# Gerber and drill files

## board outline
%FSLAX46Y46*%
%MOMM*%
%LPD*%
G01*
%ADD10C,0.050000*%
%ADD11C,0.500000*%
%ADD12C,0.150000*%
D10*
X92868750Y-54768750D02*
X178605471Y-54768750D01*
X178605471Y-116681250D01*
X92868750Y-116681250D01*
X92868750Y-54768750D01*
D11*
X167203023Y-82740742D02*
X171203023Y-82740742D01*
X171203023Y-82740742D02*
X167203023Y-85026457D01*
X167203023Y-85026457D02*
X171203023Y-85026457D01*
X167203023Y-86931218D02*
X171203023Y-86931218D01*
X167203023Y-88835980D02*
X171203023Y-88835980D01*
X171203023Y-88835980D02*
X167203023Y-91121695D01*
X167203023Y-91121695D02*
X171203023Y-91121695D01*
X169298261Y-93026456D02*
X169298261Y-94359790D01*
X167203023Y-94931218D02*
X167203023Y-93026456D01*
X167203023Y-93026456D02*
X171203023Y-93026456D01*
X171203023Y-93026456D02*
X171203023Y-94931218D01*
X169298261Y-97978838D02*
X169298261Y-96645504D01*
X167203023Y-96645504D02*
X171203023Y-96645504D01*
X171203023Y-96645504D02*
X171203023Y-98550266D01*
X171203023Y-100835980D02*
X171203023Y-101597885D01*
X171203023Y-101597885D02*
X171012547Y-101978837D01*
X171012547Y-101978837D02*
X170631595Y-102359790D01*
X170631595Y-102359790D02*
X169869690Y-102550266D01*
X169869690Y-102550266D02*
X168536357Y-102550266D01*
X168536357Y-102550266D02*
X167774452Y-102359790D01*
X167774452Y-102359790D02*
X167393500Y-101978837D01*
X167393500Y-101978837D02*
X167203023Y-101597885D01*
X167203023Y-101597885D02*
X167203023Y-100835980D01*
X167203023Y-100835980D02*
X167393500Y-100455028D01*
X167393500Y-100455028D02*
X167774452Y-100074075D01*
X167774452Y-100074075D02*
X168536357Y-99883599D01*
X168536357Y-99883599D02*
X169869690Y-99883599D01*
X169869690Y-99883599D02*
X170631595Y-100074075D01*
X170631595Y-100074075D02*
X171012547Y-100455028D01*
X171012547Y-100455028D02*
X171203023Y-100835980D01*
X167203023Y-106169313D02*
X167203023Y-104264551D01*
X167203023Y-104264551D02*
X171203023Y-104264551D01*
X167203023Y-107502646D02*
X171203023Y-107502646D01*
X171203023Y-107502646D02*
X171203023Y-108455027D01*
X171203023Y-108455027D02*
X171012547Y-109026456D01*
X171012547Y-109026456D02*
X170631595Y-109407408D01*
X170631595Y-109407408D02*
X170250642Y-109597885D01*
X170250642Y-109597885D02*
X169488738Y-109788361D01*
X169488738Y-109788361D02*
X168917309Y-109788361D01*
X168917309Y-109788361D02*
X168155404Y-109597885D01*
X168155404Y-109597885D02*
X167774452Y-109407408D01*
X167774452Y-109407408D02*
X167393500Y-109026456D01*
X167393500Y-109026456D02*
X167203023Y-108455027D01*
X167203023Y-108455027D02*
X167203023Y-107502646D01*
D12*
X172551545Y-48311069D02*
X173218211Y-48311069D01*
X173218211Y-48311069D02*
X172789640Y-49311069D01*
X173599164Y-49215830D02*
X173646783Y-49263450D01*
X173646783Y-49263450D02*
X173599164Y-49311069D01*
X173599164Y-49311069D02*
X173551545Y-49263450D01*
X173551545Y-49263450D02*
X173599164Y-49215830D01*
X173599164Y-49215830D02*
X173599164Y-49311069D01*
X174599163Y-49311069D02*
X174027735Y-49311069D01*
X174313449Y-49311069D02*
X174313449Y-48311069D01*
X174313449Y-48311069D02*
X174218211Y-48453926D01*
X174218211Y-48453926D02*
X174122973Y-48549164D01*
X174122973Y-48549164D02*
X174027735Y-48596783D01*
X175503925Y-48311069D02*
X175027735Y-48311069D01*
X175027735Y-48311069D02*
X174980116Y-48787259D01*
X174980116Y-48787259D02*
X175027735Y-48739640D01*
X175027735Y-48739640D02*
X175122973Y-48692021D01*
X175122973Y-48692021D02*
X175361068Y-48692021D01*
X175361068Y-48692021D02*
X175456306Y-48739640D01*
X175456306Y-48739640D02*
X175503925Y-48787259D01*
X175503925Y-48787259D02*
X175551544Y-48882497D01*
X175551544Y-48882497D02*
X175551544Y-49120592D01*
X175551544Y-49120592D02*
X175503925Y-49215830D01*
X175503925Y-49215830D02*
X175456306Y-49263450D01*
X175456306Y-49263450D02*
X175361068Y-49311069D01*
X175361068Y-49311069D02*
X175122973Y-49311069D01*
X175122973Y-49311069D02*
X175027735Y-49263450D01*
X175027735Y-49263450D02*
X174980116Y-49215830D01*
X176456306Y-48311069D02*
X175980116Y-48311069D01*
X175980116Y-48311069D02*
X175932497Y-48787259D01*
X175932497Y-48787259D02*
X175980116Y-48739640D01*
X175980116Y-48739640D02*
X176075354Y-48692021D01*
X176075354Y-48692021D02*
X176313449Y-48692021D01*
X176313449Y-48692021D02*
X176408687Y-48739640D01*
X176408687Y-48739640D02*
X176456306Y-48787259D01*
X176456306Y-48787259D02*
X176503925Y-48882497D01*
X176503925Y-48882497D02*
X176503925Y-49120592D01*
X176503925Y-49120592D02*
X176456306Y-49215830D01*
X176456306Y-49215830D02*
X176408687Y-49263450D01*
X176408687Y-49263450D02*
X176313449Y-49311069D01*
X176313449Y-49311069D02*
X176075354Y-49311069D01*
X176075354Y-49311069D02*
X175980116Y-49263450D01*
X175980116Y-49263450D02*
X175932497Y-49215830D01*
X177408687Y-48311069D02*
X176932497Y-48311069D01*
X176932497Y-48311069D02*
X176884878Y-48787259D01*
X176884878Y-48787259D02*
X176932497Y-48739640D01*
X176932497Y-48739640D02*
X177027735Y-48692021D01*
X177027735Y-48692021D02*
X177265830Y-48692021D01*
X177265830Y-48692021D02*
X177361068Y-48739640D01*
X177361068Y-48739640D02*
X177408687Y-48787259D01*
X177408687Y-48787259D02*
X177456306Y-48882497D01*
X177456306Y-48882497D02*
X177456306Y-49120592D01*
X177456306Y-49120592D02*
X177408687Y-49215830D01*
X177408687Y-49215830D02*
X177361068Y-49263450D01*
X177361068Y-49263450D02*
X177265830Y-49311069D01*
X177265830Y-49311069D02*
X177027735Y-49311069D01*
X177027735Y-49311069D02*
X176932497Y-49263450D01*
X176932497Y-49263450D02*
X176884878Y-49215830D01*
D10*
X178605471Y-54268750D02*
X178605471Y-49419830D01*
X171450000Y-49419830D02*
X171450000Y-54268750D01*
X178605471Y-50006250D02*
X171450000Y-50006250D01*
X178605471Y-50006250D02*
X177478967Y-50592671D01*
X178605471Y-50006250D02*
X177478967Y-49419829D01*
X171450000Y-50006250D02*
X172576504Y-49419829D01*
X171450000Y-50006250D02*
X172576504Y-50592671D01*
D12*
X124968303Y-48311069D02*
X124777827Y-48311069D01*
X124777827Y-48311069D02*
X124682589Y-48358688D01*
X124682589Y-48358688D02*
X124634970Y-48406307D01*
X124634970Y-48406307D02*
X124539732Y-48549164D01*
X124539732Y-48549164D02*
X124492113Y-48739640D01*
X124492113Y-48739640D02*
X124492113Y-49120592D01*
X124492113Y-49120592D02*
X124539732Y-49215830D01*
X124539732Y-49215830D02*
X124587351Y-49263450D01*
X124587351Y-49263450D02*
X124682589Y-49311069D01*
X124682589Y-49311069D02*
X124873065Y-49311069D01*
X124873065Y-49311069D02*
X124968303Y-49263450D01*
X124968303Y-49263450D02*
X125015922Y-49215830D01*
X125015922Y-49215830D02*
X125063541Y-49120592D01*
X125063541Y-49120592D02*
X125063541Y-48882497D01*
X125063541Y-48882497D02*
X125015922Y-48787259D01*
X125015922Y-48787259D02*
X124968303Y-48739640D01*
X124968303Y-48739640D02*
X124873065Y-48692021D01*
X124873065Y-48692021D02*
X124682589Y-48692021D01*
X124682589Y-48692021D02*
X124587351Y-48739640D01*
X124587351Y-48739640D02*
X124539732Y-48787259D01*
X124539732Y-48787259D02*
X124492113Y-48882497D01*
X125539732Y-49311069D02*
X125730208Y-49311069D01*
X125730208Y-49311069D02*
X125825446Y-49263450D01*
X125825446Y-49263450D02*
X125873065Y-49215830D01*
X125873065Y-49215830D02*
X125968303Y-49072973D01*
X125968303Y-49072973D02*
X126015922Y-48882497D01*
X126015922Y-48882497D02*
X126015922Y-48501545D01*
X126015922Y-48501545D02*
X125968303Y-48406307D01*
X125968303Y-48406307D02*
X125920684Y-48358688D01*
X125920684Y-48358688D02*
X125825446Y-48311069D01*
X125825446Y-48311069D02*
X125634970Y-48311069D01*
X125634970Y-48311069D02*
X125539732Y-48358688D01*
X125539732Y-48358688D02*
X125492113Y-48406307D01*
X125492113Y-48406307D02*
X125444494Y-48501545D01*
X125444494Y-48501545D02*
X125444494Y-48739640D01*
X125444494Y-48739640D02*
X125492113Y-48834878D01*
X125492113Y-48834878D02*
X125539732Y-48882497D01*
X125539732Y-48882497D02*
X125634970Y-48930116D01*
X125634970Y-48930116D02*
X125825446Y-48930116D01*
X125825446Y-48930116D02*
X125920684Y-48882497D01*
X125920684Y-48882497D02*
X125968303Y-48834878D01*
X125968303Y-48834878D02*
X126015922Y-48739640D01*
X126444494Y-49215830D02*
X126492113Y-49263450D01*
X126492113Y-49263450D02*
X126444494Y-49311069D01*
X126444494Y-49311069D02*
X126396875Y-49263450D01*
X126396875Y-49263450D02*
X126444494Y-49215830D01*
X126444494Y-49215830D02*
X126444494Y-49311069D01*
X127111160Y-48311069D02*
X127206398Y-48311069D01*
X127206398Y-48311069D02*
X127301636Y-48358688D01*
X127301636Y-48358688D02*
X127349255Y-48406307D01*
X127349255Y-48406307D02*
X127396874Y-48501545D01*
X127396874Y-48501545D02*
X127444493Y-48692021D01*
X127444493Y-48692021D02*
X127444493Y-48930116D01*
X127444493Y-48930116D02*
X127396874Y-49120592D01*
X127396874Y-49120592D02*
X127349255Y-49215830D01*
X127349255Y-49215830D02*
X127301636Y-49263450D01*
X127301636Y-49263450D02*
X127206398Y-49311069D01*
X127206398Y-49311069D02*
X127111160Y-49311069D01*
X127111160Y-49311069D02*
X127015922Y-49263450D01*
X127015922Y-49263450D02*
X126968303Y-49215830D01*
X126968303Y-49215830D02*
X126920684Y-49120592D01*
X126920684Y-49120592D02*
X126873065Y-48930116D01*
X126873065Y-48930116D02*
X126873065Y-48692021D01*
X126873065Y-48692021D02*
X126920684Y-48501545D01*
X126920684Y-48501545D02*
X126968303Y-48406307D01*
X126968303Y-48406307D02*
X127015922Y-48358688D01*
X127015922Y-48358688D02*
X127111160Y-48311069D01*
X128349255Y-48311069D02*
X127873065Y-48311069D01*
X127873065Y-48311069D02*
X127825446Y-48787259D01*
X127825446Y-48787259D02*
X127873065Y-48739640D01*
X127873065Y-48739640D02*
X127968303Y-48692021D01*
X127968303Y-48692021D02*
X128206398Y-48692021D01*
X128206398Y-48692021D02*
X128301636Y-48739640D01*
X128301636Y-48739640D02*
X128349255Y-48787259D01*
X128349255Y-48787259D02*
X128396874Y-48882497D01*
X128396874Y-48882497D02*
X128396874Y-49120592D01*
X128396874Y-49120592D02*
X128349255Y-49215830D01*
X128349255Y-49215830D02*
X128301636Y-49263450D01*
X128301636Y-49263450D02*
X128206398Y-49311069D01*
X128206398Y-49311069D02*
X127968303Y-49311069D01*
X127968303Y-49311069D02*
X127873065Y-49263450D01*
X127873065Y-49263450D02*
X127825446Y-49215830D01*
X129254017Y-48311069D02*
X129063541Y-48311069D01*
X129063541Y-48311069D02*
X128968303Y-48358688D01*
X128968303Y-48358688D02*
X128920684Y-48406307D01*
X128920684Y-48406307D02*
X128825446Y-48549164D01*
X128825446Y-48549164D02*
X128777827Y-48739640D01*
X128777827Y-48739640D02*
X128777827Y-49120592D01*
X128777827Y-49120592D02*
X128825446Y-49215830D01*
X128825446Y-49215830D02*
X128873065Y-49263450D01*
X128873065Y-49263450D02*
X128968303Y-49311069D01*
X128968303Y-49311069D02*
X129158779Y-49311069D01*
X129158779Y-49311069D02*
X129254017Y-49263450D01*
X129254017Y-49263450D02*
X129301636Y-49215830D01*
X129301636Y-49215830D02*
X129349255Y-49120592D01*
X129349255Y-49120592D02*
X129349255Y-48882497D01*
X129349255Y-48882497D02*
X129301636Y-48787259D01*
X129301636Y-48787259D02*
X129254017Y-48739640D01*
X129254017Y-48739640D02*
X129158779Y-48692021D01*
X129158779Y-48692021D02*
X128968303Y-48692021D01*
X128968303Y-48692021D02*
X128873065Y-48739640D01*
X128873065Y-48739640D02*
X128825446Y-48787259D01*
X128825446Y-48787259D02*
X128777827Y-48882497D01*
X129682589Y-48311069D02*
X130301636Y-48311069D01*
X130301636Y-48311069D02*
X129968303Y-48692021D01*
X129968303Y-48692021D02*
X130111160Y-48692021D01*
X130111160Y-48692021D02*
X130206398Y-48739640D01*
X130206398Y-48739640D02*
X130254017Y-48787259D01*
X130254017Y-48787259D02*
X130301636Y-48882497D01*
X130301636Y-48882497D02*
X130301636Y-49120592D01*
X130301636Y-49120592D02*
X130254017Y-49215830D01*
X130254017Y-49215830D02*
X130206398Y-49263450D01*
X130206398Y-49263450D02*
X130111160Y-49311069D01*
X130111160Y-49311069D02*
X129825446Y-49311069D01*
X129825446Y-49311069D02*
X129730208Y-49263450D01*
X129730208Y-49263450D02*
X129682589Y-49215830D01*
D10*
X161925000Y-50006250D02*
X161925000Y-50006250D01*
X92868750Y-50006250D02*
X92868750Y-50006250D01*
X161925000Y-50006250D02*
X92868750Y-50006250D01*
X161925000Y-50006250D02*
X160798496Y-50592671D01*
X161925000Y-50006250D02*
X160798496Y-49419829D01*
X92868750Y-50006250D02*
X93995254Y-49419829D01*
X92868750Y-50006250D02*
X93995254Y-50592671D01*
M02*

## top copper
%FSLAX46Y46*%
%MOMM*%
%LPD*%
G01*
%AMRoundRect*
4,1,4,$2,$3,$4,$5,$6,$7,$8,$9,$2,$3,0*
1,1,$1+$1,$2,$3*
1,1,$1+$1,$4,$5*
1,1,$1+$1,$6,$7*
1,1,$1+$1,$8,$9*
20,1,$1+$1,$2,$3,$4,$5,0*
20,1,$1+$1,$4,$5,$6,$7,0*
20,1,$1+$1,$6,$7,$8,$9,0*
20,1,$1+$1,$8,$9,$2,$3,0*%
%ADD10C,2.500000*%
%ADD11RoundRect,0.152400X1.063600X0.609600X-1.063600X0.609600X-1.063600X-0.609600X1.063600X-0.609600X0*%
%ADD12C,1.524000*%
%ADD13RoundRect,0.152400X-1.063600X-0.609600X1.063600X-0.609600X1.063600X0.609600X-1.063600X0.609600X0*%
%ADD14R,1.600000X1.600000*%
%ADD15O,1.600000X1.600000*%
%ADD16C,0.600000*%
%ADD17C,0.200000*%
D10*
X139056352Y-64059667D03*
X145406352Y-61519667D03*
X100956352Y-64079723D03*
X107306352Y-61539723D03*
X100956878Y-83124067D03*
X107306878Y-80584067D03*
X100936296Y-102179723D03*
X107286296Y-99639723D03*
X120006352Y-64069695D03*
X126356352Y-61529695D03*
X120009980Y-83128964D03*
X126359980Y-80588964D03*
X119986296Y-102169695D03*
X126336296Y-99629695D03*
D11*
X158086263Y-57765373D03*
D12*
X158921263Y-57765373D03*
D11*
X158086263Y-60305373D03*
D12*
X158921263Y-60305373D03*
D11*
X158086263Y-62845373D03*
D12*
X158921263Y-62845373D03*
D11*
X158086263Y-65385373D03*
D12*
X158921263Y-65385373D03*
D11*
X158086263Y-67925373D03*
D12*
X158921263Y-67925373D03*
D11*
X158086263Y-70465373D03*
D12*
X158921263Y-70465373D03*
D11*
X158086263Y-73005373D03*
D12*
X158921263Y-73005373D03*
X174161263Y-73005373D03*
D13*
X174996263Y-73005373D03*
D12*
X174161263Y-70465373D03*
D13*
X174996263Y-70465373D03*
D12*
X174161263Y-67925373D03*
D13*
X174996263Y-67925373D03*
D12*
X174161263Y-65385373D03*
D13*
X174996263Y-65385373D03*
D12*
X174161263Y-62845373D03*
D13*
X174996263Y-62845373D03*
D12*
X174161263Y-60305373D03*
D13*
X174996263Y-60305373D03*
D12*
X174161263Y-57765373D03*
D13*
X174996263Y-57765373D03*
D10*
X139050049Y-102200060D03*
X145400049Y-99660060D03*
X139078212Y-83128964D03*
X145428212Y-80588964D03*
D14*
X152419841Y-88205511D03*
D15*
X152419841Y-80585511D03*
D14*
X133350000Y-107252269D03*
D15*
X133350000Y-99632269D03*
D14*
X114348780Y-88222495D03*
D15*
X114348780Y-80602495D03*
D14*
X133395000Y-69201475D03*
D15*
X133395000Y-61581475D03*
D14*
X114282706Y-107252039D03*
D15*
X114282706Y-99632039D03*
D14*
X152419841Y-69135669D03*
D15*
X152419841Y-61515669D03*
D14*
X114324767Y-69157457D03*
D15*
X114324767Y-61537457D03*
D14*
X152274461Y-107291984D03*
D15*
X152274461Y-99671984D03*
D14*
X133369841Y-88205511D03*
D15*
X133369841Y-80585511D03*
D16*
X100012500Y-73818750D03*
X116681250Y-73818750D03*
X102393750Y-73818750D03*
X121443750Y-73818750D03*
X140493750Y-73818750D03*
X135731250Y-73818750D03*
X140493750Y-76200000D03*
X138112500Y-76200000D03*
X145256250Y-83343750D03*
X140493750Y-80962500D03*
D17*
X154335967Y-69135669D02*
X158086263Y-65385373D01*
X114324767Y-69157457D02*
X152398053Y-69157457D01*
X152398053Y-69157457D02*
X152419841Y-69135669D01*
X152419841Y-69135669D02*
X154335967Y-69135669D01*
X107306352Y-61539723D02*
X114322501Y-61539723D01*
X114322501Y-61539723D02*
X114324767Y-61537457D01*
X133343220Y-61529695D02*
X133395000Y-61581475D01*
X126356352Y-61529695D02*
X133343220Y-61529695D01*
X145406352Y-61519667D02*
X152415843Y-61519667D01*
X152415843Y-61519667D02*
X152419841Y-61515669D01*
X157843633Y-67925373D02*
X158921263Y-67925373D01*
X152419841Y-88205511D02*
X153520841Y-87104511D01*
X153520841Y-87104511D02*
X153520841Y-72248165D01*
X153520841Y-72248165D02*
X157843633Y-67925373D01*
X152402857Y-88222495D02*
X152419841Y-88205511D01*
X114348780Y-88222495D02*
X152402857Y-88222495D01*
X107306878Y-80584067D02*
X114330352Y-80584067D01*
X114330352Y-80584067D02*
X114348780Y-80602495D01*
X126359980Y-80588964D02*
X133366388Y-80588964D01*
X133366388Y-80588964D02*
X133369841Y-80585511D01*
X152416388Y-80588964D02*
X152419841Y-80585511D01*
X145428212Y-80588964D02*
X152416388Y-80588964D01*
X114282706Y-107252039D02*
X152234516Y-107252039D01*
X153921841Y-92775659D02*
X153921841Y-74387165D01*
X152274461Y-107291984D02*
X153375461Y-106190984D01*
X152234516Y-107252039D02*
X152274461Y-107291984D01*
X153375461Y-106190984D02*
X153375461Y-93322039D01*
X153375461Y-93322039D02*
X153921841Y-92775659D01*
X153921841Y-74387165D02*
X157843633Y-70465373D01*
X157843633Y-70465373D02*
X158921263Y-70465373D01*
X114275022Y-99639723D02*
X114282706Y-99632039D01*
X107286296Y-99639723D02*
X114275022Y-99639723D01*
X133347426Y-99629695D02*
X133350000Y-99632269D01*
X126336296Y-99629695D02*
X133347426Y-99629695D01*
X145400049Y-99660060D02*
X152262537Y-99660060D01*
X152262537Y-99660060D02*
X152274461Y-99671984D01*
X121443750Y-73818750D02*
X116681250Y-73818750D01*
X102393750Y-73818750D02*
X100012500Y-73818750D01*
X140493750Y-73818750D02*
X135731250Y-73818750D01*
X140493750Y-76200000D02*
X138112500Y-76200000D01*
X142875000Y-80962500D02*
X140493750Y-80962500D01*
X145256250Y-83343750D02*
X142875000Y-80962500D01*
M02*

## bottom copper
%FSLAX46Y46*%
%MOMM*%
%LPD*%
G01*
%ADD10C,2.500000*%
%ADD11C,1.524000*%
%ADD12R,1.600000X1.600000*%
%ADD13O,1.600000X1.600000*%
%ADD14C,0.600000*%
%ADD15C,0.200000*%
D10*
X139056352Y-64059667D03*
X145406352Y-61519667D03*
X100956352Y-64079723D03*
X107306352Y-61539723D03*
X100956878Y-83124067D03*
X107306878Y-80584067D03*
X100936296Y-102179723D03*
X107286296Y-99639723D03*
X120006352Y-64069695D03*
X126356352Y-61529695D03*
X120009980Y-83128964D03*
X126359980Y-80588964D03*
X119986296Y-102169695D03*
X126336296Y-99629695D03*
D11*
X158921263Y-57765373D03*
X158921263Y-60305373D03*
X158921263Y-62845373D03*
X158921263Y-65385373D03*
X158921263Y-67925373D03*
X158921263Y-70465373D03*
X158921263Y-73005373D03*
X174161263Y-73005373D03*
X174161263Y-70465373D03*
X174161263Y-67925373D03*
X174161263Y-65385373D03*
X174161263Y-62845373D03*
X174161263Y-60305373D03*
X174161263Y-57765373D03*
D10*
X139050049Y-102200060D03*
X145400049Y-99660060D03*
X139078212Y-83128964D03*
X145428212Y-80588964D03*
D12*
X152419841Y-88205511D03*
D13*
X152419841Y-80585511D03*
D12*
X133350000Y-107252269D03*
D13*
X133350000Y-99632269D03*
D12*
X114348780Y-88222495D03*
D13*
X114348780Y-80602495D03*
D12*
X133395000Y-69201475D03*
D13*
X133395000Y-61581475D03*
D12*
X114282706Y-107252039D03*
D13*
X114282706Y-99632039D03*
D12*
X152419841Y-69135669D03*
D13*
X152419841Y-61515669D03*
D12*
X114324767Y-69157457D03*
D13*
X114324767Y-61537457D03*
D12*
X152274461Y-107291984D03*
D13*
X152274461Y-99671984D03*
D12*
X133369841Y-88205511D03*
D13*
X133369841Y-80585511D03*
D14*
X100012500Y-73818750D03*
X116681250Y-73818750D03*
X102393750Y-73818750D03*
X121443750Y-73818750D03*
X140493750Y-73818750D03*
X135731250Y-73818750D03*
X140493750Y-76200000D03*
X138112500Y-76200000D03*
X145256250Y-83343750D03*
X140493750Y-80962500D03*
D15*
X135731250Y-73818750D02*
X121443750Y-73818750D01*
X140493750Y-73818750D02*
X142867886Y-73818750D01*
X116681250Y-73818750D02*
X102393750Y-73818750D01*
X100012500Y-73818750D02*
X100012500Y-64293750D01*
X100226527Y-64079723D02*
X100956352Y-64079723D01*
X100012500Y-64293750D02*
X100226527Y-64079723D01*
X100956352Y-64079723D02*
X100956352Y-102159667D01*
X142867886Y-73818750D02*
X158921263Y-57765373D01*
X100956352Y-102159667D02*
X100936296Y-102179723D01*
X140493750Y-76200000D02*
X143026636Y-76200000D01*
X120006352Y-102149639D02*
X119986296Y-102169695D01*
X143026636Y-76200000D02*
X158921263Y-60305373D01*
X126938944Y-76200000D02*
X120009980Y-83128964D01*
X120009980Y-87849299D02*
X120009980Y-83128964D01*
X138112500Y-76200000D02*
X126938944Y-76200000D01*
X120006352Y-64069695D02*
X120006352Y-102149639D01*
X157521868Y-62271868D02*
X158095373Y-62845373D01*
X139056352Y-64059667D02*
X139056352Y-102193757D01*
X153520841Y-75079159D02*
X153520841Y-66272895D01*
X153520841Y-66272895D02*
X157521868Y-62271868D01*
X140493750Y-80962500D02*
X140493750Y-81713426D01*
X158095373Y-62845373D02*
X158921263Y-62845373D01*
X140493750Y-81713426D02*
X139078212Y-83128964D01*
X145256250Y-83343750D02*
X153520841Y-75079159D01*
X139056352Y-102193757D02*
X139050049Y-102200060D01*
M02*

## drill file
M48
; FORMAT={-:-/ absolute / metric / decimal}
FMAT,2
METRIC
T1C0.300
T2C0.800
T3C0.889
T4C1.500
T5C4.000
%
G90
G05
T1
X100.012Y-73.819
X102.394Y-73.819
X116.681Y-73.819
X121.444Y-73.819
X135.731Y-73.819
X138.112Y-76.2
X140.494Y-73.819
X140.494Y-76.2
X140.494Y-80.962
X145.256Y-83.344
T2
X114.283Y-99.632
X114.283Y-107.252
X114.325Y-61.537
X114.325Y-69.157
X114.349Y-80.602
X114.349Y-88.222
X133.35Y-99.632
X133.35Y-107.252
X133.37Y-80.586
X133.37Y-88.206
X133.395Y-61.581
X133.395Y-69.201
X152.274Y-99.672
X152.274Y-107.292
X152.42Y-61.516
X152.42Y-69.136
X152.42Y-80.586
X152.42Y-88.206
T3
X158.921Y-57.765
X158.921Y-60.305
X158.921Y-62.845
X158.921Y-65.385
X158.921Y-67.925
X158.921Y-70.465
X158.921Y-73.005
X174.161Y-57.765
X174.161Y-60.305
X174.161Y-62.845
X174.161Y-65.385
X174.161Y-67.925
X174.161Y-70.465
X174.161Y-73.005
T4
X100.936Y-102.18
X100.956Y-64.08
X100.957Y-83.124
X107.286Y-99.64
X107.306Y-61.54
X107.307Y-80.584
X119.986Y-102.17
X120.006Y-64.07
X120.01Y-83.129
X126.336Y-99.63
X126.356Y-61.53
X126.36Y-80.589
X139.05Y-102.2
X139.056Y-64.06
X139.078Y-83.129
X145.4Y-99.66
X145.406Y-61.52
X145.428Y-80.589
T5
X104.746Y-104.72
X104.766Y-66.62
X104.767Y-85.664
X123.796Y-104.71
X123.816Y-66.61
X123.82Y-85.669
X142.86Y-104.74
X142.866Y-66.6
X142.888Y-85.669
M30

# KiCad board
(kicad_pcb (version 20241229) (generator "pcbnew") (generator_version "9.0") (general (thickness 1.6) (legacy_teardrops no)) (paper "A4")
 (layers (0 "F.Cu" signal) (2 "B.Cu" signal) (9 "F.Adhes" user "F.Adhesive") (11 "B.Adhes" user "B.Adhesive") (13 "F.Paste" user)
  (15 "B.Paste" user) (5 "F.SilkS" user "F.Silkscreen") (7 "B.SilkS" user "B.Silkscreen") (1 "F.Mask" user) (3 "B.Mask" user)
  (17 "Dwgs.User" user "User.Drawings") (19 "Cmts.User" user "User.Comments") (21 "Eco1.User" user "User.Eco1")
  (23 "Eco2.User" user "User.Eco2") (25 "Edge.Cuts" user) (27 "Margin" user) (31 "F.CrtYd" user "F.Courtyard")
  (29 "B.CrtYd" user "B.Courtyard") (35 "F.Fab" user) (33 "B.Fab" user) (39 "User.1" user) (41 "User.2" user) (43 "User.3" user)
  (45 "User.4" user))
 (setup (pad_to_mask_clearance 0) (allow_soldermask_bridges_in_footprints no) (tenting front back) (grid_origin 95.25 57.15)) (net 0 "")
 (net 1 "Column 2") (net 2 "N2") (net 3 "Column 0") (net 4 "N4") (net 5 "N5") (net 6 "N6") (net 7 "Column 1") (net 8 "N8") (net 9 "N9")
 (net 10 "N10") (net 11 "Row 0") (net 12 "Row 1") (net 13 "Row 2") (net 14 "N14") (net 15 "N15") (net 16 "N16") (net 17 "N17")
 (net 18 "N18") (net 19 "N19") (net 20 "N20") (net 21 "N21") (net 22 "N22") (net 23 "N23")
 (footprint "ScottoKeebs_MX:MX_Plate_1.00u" (layer "F.Cu") (at 142.866352 66.599667)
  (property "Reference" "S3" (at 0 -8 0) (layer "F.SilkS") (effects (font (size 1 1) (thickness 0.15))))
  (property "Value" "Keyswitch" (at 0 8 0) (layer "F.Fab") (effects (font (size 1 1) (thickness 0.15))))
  (pad "" np_thru_hole circle (at 0 0) (size 4 4) (drill 4) (layers "*.Cu" "*.Mask"))
  (pad "1" thru_hole circle (at -3.81 -2.54) (size 2.5 2.5) (drill 1.5) (layers "*.Cu" "*.Mask") (remove_unused_layers no)
   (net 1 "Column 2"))
  (pad "2" thru_hole circle (at 2.54 -5.08) (size 2.5 2.5) (drill 1.5) (layers "*.Cu" "*.Mask") (remove_unused_layers no) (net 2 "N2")))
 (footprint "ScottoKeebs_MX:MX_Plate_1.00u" (layer "F.Cu") (at 104.766352 66.619723)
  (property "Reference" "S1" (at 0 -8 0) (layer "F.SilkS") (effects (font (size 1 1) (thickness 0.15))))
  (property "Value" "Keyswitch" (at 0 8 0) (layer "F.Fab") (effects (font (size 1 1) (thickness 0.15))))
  (pad "" np_thru_hole circle (at 0 0) (size 4 4) (drill 4) (layers "*.Cu" "*.Mask"))
  (pad "1" thru_hole circle (at -3.81 -2.54) (size 2.5 2.5) (drill 1.5) (layers "*.Cu" "*.Mask") (remove_unused_layers no)
   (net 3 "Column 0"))
  (pad "2" thru_hole circle (at 2.54 -5.08) (size 2.5 2.5) (drill 1.5) (layers "*.Cu" "*.Mask") (remove_unused_layers no) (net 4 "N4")))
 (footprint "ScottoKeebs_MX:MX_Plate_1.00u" (layer "F.Cu") (at 104.766878 85.664067)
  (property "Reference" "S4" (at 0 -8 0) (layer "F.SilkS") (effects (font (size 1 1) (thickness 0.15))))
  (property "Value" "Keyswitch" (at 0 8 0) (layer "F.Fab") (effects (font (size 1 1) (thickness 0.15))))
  (pad "" np_thru_hole circle (at 0 0) (size 4 4) (drill 4) (layers "*.Cu" "*.Mask"))
  (pad "1" thru_hole circle (at -3.81 -2.54) (size 2.5 2.5) (drill 1.5) (layers "*.Cu" "*.Mask") (remove_unused_layers no)
   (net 3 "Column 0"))
  (pad "2" thru_hole circle (at 2.54 -5.08) (size 2.5 2.5) (drill 1.5) (layers "*.Cu" "*.Mask") (remove_unused_layers no) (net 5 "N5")))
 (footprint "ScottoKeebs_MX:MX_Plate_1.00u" (layer "F.Cu") (at 104.746296 104.719723)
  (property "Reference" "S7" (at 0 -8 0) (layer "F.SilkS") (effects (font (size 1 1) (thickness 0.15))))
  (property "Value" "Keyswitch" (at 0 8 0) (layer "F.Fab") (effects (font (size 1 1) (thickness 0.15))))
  (pad "" np_thru_hole circle (at 0 0) (size 4 4) (drill 4) (layers "*.Cu" "*.Mask"))
  (pad "1" thru_hole circle (at -3.81 -2.54) (size 2.5 2.5) (drill 1.5) (layers "*.Cu" "*.Mask") (remove_unused_layers no)
   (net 3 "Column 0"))
  (pad "2" thru_hole circle (at 2.54 -5.08) (size 2.5 2.5) (drill 1.5) (layers "*.Cu" "*.Mask") (remove_unused_layers no) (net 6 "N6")))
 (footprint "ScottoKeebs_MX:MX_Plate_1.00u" (layer "F.Cu") (at 123.816352 66.609695)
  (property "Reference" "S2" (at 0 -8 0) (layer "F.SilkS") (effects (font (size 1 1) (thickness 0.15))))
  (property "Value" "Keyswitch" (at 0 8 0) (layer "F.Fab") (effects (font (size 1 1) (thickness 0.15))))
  (pad "" np_thru_hole circle (at 0 0) (size 4 4) (drill 4) (layers "*.Cu" "*.Mask"))
  (pad "1" thru_hole circle (at -3.81 -2.54) (size 2.5 2.5) (drill 1.5) (layers "*.Cu" "*.Mask") (remove_unused_layers no)
   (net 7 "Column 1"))
  (pad "2" thru_hole circle (at 2.54 -5.08) (size 2.5 2.5) (drill 1.5) (layers "*.Cu" "*.Mask") (remove_unused_layers no) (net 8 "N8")))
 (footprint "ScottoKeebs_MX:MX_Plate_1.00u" (layer "F.Cu") (at 123.81998 85.668964)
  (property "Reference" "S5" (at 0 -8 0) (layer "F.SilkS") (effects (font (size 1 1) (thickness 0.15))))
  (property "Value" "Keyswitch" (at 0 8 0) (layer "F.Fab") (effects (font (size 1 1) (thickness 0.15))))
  (pad "" np_thru_hole circle (at 0 0) (size 4 4) (drill 4) (layers "*.Cu" "*.Mask"))
  (pad "1" thru_hole circle (at -3.81 -2.54) (size 2.5 2.5) (drill 1.5) (layers "*.Cu" "*.Mask") (remove_unused_layers no)
   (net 7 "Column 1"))
  (pad "2" thru_hole circle (at 2.54 -5.08) (size 2.5 2.5) (drill 1.5) (layers "*.Cu" "*.Mask") (remove_unused_layers no) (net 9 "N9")))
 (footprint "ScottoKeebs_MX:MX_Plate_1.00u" (layer "F.Cu") (at 123.796296 104.709695)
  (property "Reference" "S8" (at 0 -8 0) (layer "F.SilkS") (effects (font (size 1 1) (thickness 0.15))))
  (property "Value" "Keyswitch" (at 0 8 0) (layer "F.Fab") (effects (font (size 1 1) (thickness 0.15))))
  (pad "" np_thru_hole circle (at 0 0) (size 4 4) (drill 4) (layers "*.Cu" "*.Mask"))
  (pad "1" thru_hole circle (at -3.81 -2.54) (size 2.5 2.5) (drill 1.5) (layers "*.Cu" "*.Mask") (remove_unused_layers no)
   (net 7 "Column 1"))
  (pad "2" thru_hole circle (at 2.54 -5.08) (size 2.5 2.5) (drill 1.5) (layers "*.Cu" "*.Mask") (remove_unused_layers no) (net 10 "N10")))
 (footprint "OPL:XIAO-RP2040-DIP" (layer "F.Cu") (at 166.541263 65.385373)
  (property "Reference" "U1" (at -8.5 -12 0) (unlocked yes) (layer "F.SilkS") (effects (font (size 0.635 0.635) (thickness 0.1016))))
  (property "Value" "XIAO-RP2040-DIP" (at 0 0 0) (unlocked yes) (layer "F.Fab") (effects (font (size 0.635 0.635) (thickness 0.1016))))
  (pad "1" smd roundrect (at -8.455 -7.62 180) (size 2.432 1.524) (layers "F.Cu" "F.Mask") (roundrect_rratio 0.1) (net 3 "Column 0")
   (thermal_bridge_angle 45))
  (pad "1" thru_hole circle (at -7.62 -7.62 180) (size 1.524 1.524) (drill 0.889) (layers "*.Cu" "*.Mask") (remove_unused_layers no)
   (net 3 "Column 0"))
  (pad "2" smd roundrect (at -8.455 -5.08 180) (size 2.432 1.524) (layers "F.Cu" "F.Mask") (roundrect_rratio 0.1) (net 7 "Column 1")
   (thermal_bridge_angle 45))
  (pad "2" thru_hole circle (at -7.62 -5.08 180) (size 1.524 1.524) (drill 0.889) (layers "*.Cu" "*.Mask") (remove_unused_layers no)
   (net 7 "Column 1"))
  (pad "3" smd roundrect (at -8.455 -2.54 180) (size 2.432 1.524) (layers "F.Cu" "F.Mask") (roundrect_rratio 0.1) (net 1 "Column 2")
   (thermal_bridge_angle 45))
  (pad "3" thru_hole circle (at -7.62 -2.54 180) (size 1.524 1.524) (drill 0.889) (layers "*.Cu" "*.Mask") (remove_unused_layers no)
   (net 1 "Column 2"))
  (pad "4" smd roundrect (at -8.455 0 180) (size 2.432 1.524) (layers "F.Cu" "F.Mask") (roundrect_rratio 0.1) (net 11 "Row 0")
   (thermal_bridge_angle 45))
  (pad "4" thru_hole circle (at -7.62 0 180) (size 1.524 1.524) (drill 0.889) (layers "*.Cu" "*.Mask") (remove_unused_layers no)
   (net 11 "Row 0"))
  (pad "5" smd roundrect (at -8.455 2.54 180) (size 2.432 1.524) (layers "F.Cu" "F.Mask") (roundrect_rratio 0.1) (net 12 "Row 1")
   (thermal_bridge_angle 45))
  (pad "5" thru_hole circle (at -7.62 2.54 180) (size 1.524 1.524) (drill 0.889) (layers "*.Cu" "*.Mask") (remove_unused_layers no)
   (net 12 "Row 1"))
  (pad "6" smd roundrect (at -8.455 5.08 180) (size 2.432 1.524) (layers "F.Cu" "F.Mask") (roundrect_rratio 0.1) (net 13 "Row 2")
   (thermal_bridge_angle 45))
  (pad "6" thru_hole circle (at -7.62 5.08 180) (size 1.524 1.524) (drill 0.889) (layers "*.Cu" "*.Mask") (remove_unused_layers no)
   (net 13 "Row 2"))
  (pad "7" smd roundrect (at -8.455 7.62 180) (size 2.432 1.524) (layers "F.Cu" "F.Mask") (roundrect_rratio 0.1) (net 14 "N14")
   (thermal_bridge_angle 45))
  (pad "7" thru_hole circle (at -7.62 7.62 180) (size 1.524 1.524) (drill 0.889) (layers "*.Cu" "*.Mask") (remove_unused_layers no)
   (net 14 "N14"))
  (pad "8" thru_hole circle (at 7.62 7.62) (size 1.524 1.524) (drill 0.889) (layers "*.Cu" "*.Mask") (remove_unused_layers no)
   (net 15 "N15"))
  (pad "8" smd roundrect (at 8.455 7.62) (size 2.432 1.524) (layers "F.Cu" "F.Mask") (roundrect_rratio 0.1) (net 15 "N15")
   (thermal_bridge_angle 45))
  (pad "9" thru_hole circle (at 7.62 5.08) (size 1.524 1.524) (drill 0.889) (layers "*.Cu" "*.Mask") (remove_unused_layers no)
   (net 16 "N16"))
  (pad "9" smd roundrect (at 8.455 5.08) (size 2.432 1.524) (layers "F.Cu" "F.Mask") (roundrect_rratio 0.1) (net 16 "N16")
   (thermal_bridge_angle 45))
  (pad "10" thru_hole circle (at 7.62 2.54) (size 1.524 1.524) (drill 0.889) (layers "*.Cu" "*.Mask") (remove_unused_layers no)
   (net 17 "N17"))
  (pad "10" smd roundrect (at 8.455 2.54) (size 2.432 1.524) (layers "F.Cu" "F.Mask") (roundrect_rratio 0.1) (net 17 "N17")
   (thermal_bridge_angle 45))
  (pad "11" thru_hole circle (at 7.62 0) (size 1.524 1.524) (drill 0.889) (layers "*.Cu" "*.Mask") (remove_unused_layers no) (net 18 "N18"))
  (pad "11" smd roundrect (at 8.455 0) (size 2.432 1.524) (layers "F.Cu" "F.Mask") (roundrect_rratio 0.1) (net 18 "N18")
   (thermal_bridge_angle 45))
  (pad "12" thru_hole circle (at 7.62 -2.54) (size 1.524 1.524) (drill 0.889) (layers "*.Cu" "*.Mask") (remove_unused_layers no)
   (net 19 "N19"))
  (pad "12" smd roundrect (at 8.455 -2.54) (size 2.432 1.524) (layers "F.Cu" "F.Mask") (roundrect_rratio 0.1) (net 19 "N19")
   (thermal_bridge_angle 45))
  (pad "13" thru_hole circle (at 7.62 -5.08) (size 1.524 1.524) (drill 0.889) (layers "*.Cu" "*.Mask") (remove_unused_layers no)
   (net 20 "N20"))
  (pad "13" smd roundrect (at 8.455 -5.08) (size 2.432 1.524) (layers "F.Cu" "F.Mask") (roundrect_rratio 0.1) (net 20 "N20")
   (thermal_bridge_angle 45))
  (pad "14" thru_hole circle (at 7.62 -7.62) (size 1.524 1.524) (drill 0.889) (layers "*.Cu" "*.Mask") (remove_unused_layers no)
   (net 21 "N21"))
  (pad "14" smd roundrect (at 8.455 -7.62) (size 2.432 1.524) (layers "F.Cu" "F.Mask") (roundrect_rratio 0.1) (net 21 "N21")
   (thermal_bridge_angle 45)))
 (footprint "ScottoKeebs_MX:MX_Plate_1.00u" (layer "F.Cu") (at 142.860049 104.74006)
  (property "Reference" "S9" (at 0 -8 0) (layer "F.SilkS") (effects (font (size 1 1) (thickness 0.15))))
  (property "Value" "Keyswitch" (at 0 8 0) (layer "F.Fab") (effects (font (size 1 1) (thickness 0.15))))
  (pad "" np_thru_hole circle (at 0 0) (size 4 4) (drill 4) (layers "*.Cu" "*.Mask"))
  (pad "1" thru_hole circle (at -3.81 -2.54) (size 2.5 2.5) (drill 1.5) (layers "*.Cu" "*.Mask") (remove_unused_layers no)
   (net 1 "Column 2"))
  (pad "2" thru_hole circle (at 2.54 -5.08) (size 2.5 2.5) (drill 1.5) (layers "*.Cu" "*.Mask") (remove_unused_layers no) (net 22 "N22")))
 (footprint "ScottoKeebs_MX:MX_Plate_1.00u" (layer "F.Cu") (at 142.888212 85.668964)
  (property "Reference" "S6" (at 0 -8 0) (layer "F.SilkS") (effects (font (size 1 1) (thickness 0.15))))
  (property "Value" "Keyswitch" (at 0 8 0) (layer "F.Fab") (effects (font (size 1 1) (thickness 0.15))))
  (pad "" np_thru_hole circle (at 0 0) (size 4 4) (drill 4) (layers "*.Cu" "*.Mask"))
  (pad "1" thru_hole circle (at -3.81 -2.54) (size 2.5 2.5) (drill 1.5) (layers "*.Cu" "*.Mask") (remove_unused_layers no)
   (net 1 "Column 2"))
  (pad "2" thru_hole circle (at 2.54 -5.08) (size 2.5 2.5) (drill 1.5) (layers "*.Cu" "*.Mask") (remove_unused_layers no) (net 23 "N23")))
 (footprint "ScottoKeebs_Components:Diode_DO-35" (layer "B.Cu") (at 152.419841 88.205511 90)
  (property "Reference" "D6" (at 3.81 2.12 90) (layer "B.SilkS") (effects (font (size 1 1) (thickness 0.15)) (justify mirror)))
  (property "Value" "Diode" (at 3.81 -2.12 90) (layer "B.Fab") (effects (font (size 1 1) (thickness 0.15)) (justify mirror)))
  (pad "1" thru_hole rect (at 0 0 90) (size 1.6 1.6) (drill 0.8) (layers "*.Cu" "*.Mask") (remove_unused_layers no) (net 12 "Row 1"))
  (pad "2" thru_hole oval (at 7.62 0 90) (size 1.6 1.6) (drill 0.8) (layers "*.Cu" "*.Mask") (remove_unused_layers no) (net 23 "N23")))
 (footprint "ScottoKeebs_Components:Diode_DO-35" (layer "B.Cu") (at 133.35 107.252269 90)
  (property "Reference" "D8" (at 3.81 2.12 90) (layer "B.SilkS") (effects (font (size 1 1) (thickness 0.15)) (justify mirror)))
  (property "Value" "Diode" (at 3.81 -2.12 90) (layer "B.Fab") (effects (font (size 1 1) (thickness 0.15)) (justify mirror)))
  (pad "1" thru_hole rect (at 0 0 90) (size 1.6 1.6) (drill 0.8) (layers "*.Cu" "*.Mask") (remove_unused_layers no) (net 13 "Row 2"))
  (pad "2" thru_hole oval (at 7.62 0 90) (size 1.6 1.6) (drill 0.8) (layers "*.Cu" "*.Mask") (remove_unused_layers no) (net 10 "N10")))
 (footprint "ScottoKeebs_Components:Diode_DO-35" (layer "B.Cu") (at 114.34878 88.222495 90)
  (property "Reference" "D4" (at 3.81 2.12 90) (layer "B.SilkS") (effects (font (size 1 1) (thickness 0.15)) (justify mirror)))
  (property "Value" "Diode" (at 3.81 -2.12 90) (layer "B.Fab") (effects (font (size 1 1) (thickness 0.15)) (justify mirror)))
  (pad "1" thru_hole rect (at 0 0 90) (size 1.6 1.6) (drill 0.8) (layers "*.Cu" "*.Mask") (remove_unused_layers no) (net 12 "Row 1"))
  (pad "2" thru_hole oval (at 7.62 0 90) (size 1.6 1.6) (drill 0.8) (layers "*.Cu" "*.Mask") (remove_unused_layers no) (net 5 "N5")))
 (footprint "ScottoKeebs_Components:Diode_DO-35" (layer "B.Cu") (at 133.395 69.201475 90)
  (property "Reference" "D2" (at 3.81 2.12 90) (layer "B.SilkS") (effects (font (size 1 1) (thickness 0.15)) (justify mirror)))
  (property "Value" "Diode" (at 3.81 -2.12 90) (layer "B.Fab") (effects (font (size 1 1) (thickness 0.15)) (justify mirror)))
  (pad "1" thru_hole rect (at 0 0 90) (size 1.6 1.6) (drill 0.8) (layers "*.Cu" "*.Mask") (remove_unused_layers no) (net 11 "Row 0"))
  (pad "2" thru_hole oval (at 7.62 0 90) (size 1.6 1.6) (drill 0.8) (layers "*.Cu" "*.Mask") (remove_unused_layers no) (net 8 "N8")))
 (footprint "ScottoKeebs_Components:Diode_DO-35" (layer "B.Cu") (at 114.282706 107.252039 90)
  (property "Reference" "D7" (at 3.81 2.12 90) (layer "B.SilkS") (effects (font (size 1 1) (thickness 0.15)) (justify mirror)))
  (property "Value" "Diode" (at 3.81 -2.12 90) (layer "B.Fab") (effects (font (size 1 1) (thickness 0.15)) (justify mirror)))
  (pad "1" thru_hole rect (at 0 0 90) (size 1.6 1.6) (drill 0.8) (layers "*.Cu" "*.Mask") (remove_unused_layers no) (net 13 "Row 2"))
  (pad "2" thru_hole oval (at 7.62 0 90) (size 1.6 1.6) (drill 0.8) (layers "*.Cu" "*.Mask") (remove_unused_layers no) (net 6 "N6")))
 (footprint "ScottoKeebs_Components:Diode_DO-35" (layer "B.Cu") (at 152.419841 69.135669 90)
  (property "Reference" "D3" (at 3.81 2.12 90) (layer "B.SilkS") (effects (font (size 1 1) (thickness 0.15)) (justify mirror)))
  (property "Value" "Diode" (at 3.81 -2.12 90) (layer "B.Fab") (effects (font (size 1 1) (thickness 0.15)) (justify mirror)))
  (pad "1" thru_hole rect (at 0 0 90) (size 1.6 1.6) (drill 0.8) (layers "*.Cu" "*.Mask") (remove_unused_layers no) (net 11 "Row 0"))
  (pad "2" thru_hole oval (at 7.62 0 90) (size 1.6 1.6) (drill 0.8) (layers "*.Cu" "*.Mask") (remove_unused_layers no) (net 2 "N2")))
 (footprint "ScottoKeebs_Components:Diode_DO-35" (layer "B.Cu") (at 114.324767 69.157457 90)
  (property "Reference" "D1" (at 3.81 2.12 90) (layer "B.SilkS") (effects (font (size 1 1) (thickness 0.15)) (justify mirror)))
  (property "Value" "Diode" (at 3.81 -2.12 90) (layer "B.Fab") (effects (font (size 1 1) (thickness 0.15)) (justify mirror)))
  (pad "1" thru_hole rect (at 0 0 90) (size 1.6 1.6) (drill 0.8) (layers "*.Cu" "*.Mask") (remove_unused_layers no) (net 11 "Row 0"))
  (pad "2" thru_hole oval (at 7.62 0 90) (size 1.6 1.6) (drill 0.8) (layers "*.Cu" "*.Mask") (remove_unused_layers no) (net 4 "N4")))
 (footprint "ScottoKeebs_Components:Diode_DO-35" (layer "B.Cu") (at 152.274461 107.291984 90)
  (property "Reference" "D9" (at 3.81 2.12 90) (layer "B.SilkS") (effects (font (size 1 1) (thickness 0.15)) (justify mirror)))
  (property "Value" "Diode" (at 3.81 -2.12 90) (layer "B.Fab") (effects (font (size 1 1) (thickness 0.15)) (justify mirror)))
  (pad "1" thru_hole rect (at 0 0 90) (size 1.6 1.6) (drill 0.8) (layers "*.Cu" "*.Mask") (remove_unused_layers no) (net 13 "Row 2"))
  (pad "2" thru_hole oval (at 7.62 0 90) (size 1.6 1.6) (drill 0.8) (layers "*.Cu" "*.Mask") (remove_unused_layers no) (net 22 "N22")))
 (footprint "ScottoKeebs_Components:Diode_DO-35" (layer "B.Cu") (at 133.369841 88.205511 90)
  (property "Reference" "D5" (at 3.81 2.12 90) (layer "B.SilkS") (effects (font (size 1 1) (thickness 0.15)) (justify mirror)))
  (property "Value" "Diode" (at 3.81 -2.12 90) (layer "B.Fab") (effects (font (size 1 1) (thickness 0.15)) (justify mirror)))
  (pad "1" thru_hole rect (at 0 0 90) (size 1.6 1.6) (drill 0.8) (layers "*.Cu" "*.Mask") (remove_unused_layers no) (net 12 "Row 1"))
  (pad "2" thru_hole oval (at 7.62 0 90) (size 1.6 1.6) (drill 0.8) (layers "*.Cu" "*.Mask") (remove_unused_layers no) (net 9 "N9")))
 (gr_rect (start 92.86875 54.76875) (end 178.605471 116.68125) (stroke (width 0.05) (type default)) (fill no) (layer "Edge.Cuts"))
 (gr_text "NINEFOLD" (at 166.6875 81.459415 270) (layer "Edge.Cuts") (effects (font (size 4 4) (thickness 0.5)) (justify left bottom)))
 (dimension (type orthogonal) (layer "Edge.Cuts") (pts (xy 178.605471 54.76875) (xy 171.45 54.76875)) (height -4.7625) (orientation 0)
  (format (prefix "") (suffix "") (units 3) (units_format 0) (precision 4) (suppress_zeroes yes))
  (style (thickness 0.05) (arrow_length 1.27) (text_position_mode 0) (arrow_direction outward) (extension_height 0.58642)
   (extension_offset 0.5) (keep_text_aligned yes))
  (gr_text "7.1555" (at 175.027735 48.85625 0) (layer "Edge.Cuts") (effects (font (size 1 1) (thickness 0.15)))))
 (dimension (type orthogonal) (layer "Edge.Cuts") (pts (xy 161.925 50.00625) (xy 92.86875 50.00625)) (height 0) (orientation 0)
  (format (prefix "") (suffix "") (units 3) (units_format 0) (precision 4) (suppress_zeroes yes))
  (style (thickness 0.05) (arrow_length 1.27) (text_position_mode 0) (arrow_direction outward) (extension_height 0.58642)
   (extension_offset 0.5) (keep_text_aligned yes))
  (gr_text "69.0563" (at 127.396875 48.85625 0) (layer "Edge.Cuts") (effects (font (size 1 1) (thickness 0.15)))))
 (segment (start 154.335967 69.135669) (end 158.086263 65.385373) (width 0.2) (layer "F.Cu") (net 11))
 (segment (start 114.324767 69.157457) (end 152.398053 69.157457) (width 0.2) (layer "F.Cu") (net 11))
 (segment (start 152.398053 69.157457) (end 152.419841 69.135669) (width 0.2) (layer "F.Cu") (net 11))
 (segment (start 152.419841 69.135669) (end 154.335967 69.135669) (width 0.2) (layer "F.Cu") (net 11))
 (segment (start 107.306352 61.539723) (end 114.322501 61.539723) (width 0.2) (layer "F.Cu") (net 4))
 (segment (start 114.322501 61.539723) (end 114.324767 61.537457) (width 0.2) (layer "F.Cu") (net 4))
 (segment (start 133.34322 61.529695) (end 133.395 61.581475) (width 0.2) (layer "F.Cu") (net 8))
 (segment (start 126.356352 61.529695) (end 133.34322 61.529695) (width 0.2) (layer "F.Cu") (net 8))
 (segment (start 145.406352 61.519667) (end 152.415843 61.519667) (width 0.2) (layer "F.Cu") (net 2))
 (segment (start 152.415843 61.519667) (end 152.419841 61.515669) (width 0.2) (layer "F.Cu") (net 2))
 (segment (start 157.843633 67.925373) (end 158.921263 67.925373) (width 0.2) (layer "F.Cu") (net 12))
 (segment (start 152.419841 88.205511) (end 153.520841 87.104511) (width 0.2) (layer "F.Cu") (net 12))
 (segment (start 153.520841 87.104511) (end 153.520841 72.248165) (width 0.2) (layer "F.Cu") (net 12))
 (segment (start 153.520841 72.248165) (end 157.843633 67.925373) (width 0.2) (layer "F.Cu") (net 12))
 (segment (start 152.402857 88.222495) (end 152.419841 88.205511) (width 0.2) (layer "F.Cu") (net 12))
 (segment (start 114.34878 88.222495) (end 152.402857 88.222495) (width 0.2) (layer "F.Cu") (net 12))
 (segment (start 107.306878 80.584067) (end 114.330352 80.584067) (width 0.2) (layer "F.Cu") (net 5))
 (segment (start 114.330352 80.584067) (end 114.34878 80.602495) (width 0.2) (layer "F.Cu") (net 5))
 (segment (start 126.35998 80.588964) (end 133.366388 80.588964) (width 0.2) (layer "F.Cu") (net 9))
 (segment (start 133.366388 80.588964) (end 133.369841 80.585511) (width 0.2) (layer "F.Cu") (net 9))
 (segment (start 152.416388 80.588964) (end 152.419841 80.585511) (width 0.2) (layer "F.Cu") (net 23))
 (segment (start 145.428212 80.588964) (end 152.416388 80.588964) (width 0.2) (layer "F.Cu") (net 23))
 (segment (start 114.282706 107.252039) (end 152.234516 107.252039) (width 0.2) (layer "F.Cu") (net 13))
 (segment (start 153.921841 92.775659) (end 153.921841 74.387165) (width 0.2) (layer "F.Cu") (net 13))
 (segment (start 152.274461 107.291984) (end 153.375461 106.190984) (width 0.2) (layer "F.Cu") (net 13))
 (segment (start 152.234516 107.252039) (end 152.274461 107.291984) (width 0.2) (layer "F.Cu") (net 13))
 (segment (start 153.375461 106.190984) (end 153.375461 93.322039) (width 0.2) (layer "F.Cu") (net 13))
 (segment (start 153.375461 93.322039) (end 153.921841 92.775659) (width 0.2) (layer "F.Cu") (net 13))
 (segment (start 153.921841 74.387165) (end 157.843633 70.465373) (width 0.2) (layer "F.Cu") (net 13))
 (segment (start 157.843633 70.465373) (end 158.921263 70.465373) (width 0.2) (layer "F.Cu") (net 13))
 (segment (start 114.275022 99.639723) (end 114.282706 99.632039) (width 0.2) (layer "F.Cu") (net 6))
 (segment (start 107.286296 99.639723) (end 114.275022 99.639723) (width 0.2) (layer "F.Cu") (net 6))
 (segment (start 133.347426 99.629695) (end 133.35 99.632269) (width 0.2) (layer "F.Cu") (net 10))
 (segment (start 126.336296 99.629695) (end 133.347426 99.629695) (width 0.2) (layer "F.Cu") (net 10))
 (segment (start 145.400049 99.66006) (end 152.262537 99.66006) (width 0.2) (layer "F.Cu") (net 22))
 (segment (start 152.262537 99.66006) (end 152.274461 99.671984) (width 0.2) (layer "F.Cu") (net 22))
 (segment (start 121.44375 73.81875) (end 116.68125 73.81875) (width 0.2) (layer "F.Cu") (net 3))
 (segment (start 102.39375 73.81875) (end 100.0125 73.81875) (width 0.2) (layer "F.Cu") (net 3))
 (segment (start 140.49375 73.81875) (end 135.73125 73.81875) (width 0.2) (layer "F.Cu") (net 3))
 (via (at 100.0125 73.81875) (size 0.6) (drill 0.3) (layers "F.Cu" "B.Cu") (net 3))
 (via (at 116.68125 73.81875) (size 0.6) (drill 0.3) (layers "F.Cu" "B.Cu") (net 3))
 (via (at 102.39375 73.81875) (size 0.6) (drill 0.3) (layers "F.Cu" "B.Cu") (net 3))
 (via (at 121.44375 73.81875) (size 0.6) (drill 0.3) (layers "F.Cu" "B.Cu") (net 3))
 (via (at 140.49375 73.81875) (size 0.6) (drill 0.3) (layers "F.Cu" "B.Cu") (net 3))
 (via (at 135.73125 73.81875) (size 0.6) (drill 0.3) (layers "F.Cu" "B.Cu") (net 3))
 (segment (start 135.73125 73.81875) (end 121.44375 73.81875) (width 0.2) (layer "B.Cu") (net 3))
 (segment (start 140.49375 73.81875) (end 142.867886 73.81875) (width 0.2) (layer "B.Cu") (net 3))
 (segment (start 116.68125 73.81875) (end 102.39375 73.81875) (width 0.2) (layer "B.Cu") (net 3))
 (segment (start 100.0125 73.81875) (end 100.0125 64.29375) (width 0.2) (layer "B.Cu") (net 3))
 (segment (start 100.226527 64.079723) (end 100.956352 64.079723) (width 0.2) (layer "B.Cu") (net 3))
 (segment (start 100.0125 64.29375) (end 100.226527 64.079723) (width 0.2) (layer "B.Cu") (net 3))
 (segment (start 100.956352 64.079723) (end 100.956352 102.159667) (width 0.2) (layer "B.Cu") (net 3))
 (segment (start 142.867886 73.81875) (end 158.921263 57.765373) (width 0.2) (layer "B.Cu") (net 3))
 (segment (start 100.956352 102.159667) (end 100.936296 102.179723) (width 0.2) (layer "B.Cu") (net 3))
 (segment (start 140.49375 76.2) (end 138.1125 76.2) (width 0.2) (layer "F.Cu") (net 7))
 (via (at 140.49375 76.2) (size 0.6) (drill 0.3) (layers "F.Cu" "B.Cu") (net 7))
 (via (at 138.1125 76.2) (size 0.6) (drill 0.3) (layers "F.Cu" "B.Cu") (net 7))
 (segment (start 140.49375 76.2) (end 143.026636 76.2) (width 0.2) (layer "B.Cu") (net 7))
 (segment (start 120.006352 102.149639) (end 119.986296 102.169695) (width 0.2) (layer "B.Cu") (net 7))
 (segment (start 143.026636 76.2) (end 158.921263 60.305373) (width 0.2) (layer "B.Cu") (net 7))
 (segment (start 126.938944 76.2) (end 120.00998 83.128964) (width 0.2) (layer "B.Cu") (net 7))
 (segment (start 120.00998 87.849299) (end 120.00998 83.128964) (width 0.2) (layer "B.Cu") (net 7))
 (segment (start 138.1125 76.2) (end 126.938944 76.2) (width 0.2) (layer "B.Cu") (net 7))
 (segment (start 120.006352 64.069695) (end 120.006352 102.149639) (width 0.2) (layer "B.Cu") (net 7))
 (segment (start 142.875 80.9625) (end 140.49375 80.9625) (width 0.2) (layer "F.Cu") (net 1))
 (segment (start 145.25625 83.34375) (end 142.875 80.9625) (width 0.2) (layer "F.Cu") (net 1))
 (via (at 145.25625 83.34375) (size 0.6) (drill 0.3) (layers "F.Cu" "B.Cu") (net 1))
 (via (at 140.49375 80.9625) (size 0.6) (drill 0.3) (layers "F.Cu" "B.Cu") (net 1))
 (segment (start 157.521868 62.271868) (end 158.095373 62.845373) (width 0.2) (layer "B.Cu") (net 1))
 (segment (start 139.056352 64.059667) (end 139.056352 102.193757) (width 0.2) (layer "B.Cu") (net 1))
 (segment (start 153.520841 75.079159) (end 153.520841 66.272895) (width 0.2) (layer "B.Cu") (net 1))
 (segment (start 153.520841 66.272895) (end 157.521868 62.271868) (width 0.2) (layer "B.Cu") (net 1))
 (segment (start 140.49375 80.9625) (end 140.49375 81.713426) (width 0.2) (layer "B.Cu") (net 1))
 (segment (start 158.095373 62.845373) (end 158.921263 62.845373) (width 0.2) (layer "B.Cu") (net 1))
 (segment (start 140.49375 81.713426) (end 139.078212 83.128964) (width 0.2) (layer "B.Cu") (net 1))
 (segment (start 145.25625 83.34375) (end 153.520841 75.079159) (width 0.2) (layer "B.Cu") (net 1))
 (segment (start 139.056352 102.193757) (end 139.050049 102.20006) (width 0.2) (layer "B.Cu") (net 1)))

